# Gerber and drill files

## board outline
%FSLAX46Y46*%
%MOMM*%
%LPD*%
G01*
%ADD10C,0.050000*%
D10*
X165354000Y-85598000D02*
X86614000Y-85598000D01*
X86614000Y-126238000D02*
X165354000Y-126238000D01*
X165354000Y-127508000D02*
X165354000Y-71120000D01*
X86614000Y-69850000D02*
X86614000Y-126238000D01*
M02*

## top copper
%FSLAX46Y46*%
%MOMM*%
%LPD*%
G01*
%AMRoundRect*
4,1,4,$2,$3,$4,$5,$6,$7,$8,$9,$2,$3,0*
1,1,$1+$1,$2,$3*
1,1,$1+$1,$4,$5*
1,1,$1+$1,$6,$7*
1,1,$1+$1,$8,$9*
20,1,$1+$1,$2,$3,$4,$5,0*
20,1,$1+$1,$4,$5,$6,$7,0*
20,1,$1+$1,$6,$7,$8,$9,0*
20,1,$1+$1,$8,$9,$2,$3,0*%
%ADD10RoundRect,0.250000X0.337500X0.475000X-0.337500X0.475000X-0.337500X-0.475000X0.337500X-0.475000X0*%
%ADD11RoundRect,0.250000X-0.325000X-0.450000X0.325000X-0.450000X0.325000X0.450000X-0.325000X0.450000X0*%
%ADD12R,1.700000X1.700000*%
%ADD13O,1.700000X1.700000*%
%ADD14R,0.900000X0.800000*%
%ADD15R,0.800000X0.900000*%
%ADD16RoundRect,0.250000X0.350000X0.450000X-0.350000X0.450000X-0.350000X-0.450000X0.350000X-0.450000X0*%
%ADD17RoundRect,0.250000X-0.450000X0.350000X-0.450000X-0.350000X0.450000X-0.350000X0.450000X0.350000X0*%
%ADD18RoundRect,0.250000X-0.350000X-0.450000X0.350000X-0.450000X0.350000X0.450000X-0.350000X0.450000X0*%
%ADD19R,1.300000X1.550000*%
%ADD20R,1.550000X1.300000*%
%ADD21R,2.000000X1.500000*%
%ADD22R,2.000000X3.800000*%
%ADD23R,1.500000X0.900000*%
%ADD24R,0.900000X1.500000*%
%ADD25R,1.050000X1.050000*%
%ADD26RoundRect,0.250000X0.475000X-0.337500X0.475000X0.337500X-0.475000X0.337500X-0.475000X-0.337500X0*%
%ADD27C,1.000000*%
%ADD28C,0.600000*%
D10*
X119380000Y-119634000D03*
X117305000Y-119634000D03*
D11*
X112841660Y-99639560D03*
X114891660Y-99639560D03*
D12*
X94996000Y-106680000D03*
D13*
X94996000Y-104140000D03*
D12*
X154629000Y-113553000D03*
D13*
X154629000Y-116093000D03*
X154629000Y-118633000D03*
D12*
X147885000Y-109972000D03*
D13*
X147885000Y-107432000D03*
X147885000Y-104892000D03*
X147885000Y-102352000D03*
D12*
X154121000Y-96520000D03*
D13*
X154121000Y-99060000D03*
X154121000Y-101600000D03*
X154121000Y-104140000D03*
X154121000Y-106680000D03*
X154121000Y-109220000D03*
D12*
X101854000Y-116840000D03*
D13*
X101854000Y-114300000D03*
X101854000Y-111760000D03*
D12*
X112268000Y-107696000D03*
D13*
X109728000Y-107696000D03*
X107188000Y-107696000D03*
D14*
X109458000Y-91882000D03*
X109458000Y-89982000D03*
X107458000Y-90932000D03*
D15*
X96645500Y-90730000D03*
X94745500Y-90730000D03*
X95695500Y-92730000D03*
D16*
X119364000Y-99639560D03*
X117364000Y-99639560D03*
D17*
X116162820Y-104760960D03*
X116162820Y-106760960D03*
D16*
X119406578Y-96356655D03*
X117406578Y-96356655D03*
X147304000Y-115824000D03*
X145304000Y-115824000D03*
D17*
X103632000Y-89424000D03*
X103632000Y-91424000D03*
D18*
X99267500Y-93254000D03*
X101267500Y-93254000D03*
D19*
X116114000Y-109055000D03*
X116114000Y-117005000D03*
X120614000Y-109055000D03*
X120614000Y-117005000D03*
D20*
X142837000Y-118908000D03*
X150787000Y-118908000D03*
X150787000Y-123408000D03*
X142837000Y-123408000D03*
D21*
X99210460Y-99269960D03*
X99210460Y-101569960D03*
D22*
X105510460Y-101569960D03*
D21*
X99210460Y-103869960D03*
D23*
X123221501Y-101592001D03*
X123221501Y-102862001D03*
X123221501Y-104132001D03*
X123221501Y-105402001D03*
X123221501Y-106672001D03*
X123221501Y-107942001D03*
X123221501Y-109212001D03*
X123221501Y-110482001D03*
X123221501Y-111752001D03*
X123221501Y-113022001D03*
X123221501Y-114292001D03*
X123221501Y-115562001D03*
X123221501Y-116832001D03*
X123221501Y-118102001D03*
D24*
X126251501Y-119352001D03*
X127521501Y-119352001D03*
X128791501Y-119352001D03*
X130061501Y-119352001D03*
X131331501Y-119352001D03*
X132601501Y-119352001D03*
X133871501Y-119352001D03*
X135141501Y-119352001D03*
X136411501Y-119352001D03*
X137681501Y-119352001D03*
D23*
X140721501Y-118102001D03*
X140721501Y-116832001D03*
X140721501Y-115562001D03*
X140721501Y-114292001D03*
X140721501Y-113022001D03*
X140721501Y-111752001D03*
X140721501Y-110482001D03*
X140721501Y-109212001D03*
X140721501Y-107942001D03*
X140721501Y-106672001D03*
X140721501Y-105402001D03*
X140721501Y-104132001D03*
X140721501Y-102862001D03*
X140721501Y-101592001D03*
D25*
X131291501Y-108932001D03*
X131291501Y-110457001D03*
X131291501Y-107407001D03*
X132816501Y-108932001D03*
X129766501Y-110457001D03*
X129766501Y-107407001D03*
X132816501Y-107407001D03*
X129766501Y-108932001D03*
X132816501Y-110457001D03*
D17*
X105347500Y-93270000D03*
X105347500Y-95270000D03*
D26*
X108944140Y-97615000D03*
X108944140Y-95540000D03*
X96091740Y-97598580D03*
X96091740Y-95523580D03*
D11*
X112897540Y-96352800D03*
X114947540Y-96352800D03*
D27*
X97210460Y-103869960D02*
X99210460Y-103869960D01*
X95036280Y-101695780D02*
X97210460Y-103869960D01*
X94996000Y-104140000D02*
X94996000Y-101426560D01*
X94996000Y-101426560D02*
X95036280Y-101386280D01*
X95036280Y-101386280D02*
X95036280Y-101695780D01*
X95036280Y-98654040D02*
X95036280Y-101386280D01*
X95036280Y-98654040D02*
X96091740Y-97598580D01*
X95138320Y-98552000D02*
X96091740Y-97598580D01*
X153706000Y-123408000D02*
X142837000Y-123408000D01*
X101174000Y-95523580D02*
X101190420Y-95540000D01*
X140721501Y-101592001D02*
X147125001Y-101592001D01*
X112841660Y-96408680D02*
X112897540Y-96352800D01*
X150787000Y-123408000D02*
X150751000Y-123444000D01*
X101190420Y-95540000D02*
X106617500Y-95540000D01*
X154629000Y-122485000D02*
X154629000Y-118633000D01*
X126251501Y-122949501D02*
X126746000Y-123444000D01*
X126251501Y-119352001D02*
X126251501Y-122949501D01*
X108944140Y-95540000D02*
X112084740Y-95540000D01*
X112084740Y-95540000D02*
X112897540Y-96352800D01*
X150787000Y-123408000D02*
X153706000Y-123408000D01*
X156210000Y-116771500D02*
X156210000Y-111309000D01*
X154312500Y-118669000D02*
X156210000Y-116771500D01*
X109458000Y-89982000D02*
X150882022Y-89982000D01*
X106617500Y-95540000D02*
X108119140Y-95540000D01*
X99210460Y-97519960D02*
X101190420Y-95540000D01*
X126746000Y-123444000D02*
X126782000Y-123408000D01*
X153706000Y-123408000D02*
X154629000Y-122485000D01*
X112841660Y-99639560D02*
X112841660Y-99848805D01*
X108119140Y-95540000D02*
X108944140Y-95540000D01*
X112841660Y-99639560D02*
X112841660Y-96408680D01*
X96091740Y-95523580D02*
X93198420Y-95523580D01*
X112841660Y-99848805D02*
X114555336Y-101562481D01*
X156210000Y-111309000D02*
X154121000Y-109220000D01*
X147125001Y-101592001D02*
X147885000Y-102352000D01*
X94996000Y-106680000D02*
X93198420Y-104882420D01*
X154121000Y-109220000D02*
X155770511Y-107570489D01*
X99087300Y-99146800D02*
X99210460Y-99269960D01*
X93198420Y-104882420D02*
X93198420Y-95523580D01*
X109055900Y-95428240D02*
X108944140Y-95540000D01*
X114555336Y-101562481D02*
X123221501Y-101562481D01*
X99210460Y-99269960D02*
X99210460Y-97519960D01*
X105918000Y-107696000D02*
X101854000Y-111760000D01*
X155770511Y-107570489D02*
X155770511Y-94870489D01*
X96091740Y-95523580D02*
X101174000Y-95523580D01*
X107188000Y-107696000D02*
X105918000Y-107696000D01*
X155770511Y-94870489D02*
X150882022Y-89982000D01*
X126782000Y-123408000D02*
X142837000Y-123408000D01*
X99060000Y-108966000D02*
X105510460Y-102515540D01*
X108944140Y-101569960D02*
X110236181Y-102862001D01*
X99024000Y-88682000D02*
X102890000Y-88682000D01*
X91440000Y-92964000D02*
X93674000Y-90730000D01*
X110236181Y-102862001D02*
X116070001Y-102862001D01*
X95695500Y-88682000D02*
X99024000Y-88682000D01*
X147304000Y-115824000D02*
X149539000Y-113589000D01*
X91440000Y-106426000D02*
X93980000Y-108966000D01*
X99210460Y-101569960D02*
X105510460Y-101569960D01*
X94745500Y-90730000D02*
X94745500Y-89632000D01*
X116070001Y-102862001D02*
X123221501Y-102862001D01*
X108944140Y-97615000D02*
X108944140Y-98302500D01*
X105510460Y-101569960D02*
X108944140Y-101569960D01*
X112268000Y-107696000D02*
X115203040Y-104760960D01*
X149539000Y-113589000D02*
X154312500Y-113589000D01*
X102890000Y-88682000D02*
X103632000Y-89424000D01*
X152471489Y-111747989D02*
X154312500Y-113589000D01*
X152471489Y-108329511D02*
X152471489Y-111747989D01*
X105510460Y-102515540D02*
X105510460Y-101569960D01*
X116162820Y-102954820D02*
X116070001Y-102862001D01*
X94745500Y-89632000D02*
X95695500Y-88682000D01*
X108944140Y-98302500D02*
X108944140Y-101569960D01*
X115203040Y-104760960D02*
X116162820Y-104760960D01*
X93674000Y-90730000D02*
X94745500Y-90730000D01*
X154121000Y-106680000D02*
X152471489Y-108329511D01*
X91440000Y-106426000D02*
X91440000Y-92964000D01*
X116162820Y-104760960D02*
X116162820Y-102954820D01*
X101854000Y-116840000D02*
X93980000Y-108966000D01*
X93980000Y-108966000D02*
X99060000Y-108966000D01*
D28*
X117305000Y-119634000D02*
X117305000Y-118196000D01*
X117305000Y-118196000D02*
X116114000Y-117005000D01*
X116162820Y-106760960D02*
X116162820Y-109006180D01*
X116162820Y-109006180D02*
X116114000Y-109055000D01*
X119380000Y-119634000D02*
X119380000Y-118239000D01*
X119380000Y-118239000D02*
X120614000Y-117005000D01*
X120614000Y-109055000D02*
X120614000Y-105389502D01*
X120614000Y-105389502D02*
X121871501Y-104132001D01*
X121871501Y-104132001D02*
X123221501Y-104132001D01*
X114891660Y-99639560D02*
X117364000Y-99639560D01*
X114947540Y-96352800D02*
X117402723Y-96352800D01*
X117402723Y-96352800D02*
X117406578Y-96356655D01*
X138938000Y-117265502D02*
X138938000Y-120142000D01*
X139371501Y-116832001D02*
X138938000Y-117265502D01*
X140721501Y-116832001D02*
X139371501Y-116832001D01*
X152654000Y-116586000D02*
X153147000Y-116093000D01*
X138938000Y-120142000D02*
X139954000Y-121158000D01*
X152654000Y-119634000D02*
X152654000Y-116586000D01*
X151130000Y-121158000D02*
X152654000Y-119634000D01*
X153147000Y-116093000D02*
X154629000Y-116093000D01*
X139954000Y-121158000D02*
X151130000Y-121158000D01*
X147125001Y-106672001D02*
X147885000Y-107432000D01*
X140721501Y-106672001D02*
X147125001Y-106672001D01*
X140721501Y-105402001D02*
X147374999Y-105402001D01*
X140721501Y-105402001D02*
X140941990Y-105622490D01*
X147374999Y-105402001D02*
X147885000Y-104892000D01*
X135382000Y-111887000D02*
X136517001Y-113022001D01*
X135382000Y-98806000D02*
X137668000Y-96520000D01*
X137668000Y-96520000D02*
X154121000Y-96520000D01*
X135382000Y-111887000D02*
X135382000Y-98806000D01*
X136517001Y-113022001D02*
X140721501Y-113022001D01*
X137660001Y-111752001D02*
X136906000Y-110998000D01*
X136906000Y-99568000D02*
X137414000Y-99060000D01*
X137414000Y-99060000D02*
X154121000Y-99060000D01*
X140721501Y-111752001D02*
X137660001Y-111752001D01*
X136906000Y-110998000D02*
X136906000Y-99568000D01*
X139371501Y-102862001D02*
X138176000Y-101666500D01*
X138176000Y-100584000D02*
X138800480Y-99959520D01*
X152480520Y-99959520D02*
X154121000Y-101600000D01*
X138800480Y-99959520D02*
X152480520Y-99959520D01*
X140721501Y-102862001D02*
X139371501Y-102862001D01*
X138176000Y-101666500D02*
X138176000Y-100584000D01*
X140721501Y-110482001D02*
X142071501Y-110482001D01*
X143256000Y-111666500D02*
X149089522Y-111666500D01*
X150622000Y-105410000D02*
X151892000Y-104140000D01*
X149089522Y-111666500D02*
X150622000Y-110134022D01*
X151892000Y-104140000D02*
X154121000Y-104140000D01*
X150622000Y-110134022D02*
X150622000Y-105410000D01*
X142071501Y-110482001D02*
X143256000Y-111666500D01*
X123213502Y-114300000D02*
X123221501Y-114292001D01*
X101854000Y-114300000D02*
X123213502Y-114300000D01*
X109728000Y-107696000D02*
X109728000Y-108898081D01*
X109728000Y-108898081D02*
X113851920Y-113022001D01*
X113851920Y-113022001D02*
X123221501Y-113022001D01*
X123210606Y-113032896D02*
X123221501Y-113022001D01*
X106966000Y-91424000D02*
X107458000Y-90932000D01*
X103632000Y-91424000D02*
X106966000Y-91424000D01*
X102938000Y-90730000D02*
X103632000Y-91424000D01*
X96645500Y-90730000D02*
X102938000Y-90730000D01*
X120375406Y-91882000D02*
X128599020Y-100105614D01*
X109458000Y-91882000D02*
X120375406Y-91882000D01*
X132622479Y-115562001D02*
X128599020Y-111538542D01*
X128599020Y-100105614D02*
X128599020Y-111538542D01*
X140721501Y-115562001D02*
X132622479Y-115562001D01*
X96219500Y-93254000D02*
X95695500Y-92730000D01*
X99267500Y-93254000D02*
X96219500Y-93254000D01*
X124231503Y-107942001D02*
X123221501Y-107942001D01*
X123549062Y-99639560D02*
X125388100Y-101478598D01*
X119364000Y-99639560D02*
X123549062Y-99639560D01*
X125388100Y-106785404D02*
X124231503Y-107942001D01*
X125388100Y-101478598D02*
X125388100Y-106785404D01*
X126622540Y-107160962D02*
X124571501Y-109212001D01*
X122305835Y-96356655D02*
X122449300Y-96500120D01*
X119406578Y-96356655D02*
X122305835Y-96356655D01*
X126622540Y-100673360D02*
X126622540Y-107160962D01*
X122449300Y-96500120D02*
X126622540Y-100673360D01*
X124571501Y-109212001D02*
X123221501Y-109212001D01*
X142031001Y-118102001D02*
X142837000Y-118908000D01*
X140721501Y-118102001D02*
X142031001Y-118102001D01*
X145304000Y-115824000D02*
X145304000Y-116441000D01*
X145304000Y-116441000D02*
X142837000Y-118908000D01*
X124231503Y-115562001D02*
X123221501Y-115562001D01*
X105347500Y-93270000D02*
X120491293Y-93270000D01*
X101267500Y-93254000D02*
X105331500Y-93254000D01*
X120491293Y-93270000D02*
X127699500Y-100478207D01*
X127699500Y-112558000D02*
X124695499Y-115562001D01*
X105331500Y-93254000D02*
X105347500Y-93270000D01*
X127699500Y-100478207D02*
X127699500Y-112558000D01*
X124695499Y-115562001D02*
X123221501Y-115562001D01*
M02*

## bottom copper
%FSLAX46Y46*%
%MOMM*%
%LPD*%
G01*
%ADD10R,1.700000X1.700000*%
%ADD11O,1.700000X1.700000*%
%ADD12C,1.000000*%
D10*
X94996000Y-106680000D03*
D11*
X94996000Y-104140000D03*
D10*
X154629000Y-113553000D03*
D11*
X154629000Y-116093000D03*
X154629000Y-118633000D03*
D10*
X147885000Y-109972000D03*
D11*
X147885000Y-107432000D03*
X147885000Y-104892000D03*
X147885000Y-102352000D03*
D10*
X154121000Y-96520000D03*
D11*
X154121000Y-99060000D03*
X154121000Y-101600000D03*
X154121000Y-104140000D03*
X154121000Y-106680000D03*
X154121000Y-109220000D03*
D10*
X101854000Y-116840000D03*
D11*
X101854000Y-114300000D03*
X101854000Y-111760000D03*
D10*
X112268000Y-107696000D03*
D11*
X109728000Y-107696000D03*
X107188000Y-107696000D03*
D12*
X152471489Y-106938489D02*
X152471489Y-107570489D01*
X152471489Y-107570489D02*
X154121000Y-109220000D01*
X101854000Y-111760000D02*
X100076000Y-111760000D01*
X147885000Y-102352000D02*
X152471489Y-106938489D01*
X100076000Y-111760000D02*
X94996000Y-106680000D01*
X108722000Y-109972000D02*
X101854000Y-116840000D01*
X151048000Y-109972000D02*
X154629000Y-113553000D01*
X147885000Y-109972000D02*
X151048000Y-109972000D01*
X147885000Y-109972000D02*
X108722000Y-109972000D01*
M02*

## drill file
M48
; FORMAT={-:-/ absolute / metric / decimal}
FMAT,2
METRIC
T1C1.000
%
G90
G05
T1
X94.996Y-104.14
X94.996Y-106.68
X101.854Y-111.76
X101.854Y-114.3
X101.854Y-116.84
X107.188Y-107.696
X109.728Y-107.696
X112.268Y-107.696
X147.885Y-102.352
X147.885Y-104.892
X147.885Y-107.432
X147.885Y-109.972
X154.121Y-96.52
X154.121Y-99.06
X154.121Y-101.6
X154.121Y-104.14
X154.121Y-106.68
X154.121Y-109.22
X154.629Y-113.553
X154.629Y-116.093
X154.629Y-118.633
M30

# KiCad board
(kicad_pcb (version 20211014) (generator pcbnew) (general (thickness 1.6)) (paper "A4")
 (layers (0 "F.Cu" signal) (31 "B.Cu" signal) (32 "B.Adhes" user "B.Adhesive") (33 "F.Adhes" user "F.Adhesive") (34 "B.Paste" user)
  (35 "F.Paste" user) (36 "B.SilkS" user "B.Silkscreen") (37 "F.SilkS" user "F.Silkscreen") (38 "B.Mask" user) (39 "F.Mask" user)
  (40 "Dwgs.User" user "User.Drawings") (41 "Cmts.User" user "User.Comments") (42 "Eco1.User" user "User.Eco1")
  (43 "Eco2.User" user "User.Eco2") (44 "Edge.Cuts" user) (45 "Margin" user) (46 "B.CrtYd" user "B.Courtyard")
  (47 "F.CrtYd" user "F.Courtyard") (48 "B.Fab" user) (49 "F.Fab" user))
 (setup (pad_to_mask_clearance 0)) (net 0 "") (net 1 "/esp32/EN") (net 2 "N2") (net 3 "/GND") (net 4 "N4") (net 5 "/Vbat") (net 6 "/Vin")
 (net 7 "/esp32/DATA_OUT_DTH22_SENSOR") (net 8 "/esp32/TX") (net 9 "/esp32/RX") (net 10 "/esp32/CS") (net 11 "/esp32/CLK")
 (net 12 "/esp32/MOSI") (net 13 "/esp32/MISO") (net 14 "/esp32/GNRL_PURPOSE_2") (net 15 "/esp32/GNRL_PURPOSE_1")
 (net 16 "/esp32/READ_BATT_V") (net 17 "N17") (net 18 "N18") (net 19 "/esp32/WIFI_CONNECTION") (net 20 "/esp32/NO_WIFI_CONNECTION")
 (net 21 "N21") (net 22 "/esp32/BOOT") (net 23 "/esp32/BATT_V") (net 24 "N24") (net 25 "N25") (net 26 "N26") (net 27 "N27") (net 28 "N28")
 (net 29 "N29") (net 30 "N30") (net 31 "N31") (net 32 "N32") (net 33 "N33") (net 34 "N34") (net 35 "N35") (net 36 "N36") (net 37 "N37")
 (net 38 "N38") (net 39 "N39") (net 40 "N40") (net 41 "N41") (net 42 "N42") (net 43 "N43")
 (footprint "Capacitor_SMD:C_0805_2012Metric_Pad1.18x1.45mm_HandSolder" (layer "F.Cu") (at 118.3425 119.634 180)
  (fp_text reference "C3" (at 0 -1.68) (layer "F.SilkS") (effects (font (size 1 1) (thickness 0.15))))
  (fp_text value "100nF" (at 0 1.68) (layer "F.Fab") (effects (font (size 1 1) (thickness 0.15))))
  (pad "1" smd roundrect locked (at -1.0375 0 180) (size 1.175 1.45) (layers "F.Cu" "F.Paste" "F.Mask") (roundrect_rratio 0.212766)
   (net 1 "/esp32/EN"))
  (pad "2" smd roundrect locked (at 1.0375 0 180) (size 1.175 1.45) (layers "F.Cu" "F.Paste" "F.Mask") (roundrect_rratio 0.212766)
   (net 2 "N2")))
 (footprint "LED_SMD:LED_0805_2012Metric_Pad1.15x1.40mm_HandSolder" (layer "F.Cu") (at 113.86666 99.63956)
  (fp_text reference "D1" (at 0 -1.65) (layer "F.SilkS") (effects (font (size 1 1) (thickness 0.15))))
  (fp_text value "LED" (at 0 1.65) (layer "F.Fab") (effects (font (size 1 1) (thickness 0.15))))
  (pad "1" smd roundrect locked (at -1.025 0) (size 1.15 1.4) (layers "F.Cu" "F.Paste" "F.Mask") (roundrect_rratio 0.217391) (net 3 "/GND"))
  (pad "2" smd roundrect locked (at 1.025 0) (size 1.15 1.4) (layers "F.Cu" "F.Paste" "F.Mask") (roundrect_rratio 0.217391) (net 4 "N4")))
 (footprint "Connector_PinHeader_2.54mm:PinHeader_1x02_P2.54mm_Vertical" (layer "F.Cu") (at 94.996 106.68 180)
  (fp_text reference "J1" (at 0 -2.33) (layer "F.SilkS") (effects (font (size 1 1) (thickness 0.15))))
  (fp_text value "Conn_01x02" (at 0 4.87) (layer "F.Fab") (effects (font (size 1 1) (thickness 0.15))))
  (pad "1" thru_hole rect locked (at 0 0 180) (size 1.7 1.7) (drill 1) (layers *.Cu *.Mask) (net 3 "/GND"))
  (pad "2" thru_hole oval locked (at 0 2.54 180) (size 1.7 1.7) (drill 1) (layers *.Cu *.Mask) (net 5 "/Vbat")))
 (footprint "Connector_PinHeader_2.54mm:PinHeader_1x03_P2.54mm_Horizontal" (layer "F.Cu") (at 154.629 113.553)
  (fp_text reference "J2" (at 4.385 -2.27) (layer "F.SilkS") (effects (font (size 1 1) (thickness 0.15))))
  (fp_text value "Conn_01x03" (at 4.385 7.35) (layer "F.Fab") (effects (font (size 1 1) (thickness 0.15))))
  (pad "1" thru_hole rect locked (at 0 0) (size 1.7 1.7) (drill 1) (layers *.Cu *.Mask) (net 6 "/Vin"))
  (pad "2" thru_hole oval locked (at 0 2.54) (size 1.7 1.7) (drill 1) (layers *.Cu *.Mask) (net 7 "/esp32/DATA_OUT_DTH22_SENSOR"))
  (pad "3" thru_hole oval locked (at 0 5.08) (size 1.7 1.7) (drill 1) (layers *.Cu *.Mask) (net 3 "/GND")))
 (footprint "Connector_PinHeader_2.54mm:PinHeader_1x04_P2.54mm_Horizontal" (layer "F.Cu") (at 147.885 109.972 180)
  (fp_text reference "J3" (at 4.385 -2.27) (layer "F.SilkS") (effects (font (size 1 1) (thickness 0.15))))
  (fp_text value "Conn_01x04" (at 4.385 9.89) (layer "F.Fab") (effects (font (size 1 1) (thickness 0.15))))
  (pad "1" thru_hole rect locked (at 0 0 180) (size 1.7 1.7) (drill 1) (layers *.Cu *.Mask) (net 6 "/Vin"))
  (pad "2" thru_hole oval locked (at 0 2.54 180) (size 1.7 1.7) (drill 1) (layers *.Cu *.Mask) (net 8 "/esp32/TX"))
  (pad "3" thru_hole oval locked (at 0 5.08 180) (size 1.7 1.7) (drill 1) (layers *.Cu *.Mask) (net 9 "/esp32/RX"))
  (pad "4" thru_hole oval locked (at 0 7.62 180) (size 1.7 1.7) (drill 1) (layers *.Cu *.Mask) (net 3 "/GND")))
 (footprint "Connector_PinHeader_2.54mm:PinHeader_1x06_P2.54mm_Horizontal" (layer "F.Cu") (at 154.121 96.52)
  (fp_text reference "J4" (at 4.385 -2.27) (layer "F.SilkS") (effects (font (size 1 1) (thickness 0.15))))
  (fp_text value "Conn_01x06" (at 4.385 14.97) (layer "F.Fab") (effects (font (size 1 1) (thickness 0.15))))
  (pad "1" thru_hole rect locked (at 0 0) (size 1.7 1.7) (drill 1) (layers *.Cu *.Mask) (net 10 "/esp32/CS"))
  (pad "2" thru_hole oval locked (at 0 2.54) (size 1.7 1.7) (drill 1) (layers *.Cu *.Mask) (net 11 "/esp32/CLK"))
  (pad "3" thru_hole oval locked (at 0 5.08) (size 1.7 1.7) (drill 1) (layers *.Cu *.Mask) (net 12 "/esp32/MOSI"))
  (pad "4" thru_hole oval locked (at 0 7.62) (size 1.7 1.7) (drill 1) (layers *.Cu *.Mask) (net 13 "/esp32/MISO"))
  (pad "5" thru_hole oval locked (at 0 10.16) (size 1.7 1.7) (drill 1) (layers *.Cu *.Mask) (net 6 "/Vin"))
  (pad "6" thru_hole oval locked (at 0 12.7) (size 1.7 1.7) (drill 1) (layers *.Cu *.Mask) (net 3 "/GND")))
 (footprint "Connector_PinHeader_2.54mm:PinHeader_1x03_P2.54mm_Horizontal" (layer "F.Cu") (at 101.854 116.84 180)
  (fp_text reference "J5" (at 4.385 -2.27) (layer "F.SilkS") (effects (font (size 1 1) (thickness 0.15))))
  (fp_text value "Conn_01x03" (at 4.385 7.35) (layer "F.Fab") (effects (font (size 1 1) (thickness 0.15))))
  (pad "1" thru_hole rect locked (at 0 0 180) (size 1.7 1.7) (drill 1) (layers *.Cu *.Mask) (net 6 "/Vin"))
  (pad "2" thru_hole oval locked (at 0 2.54 180) (size 1.7 1.7) (drill 1) (layers *.Cu *.Mask) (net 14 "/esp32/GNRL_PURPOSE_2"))
  (pad "3" thru_hole oval locked (at 0 5.08 180) (size 1.7 1.7) (drill 1) (layers *.Cu *.Mask) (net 3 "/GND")))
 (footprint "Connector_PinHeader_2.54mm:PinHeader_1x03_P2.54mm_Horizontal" (layer "F.Cu") (at 112.268 107.696 -90)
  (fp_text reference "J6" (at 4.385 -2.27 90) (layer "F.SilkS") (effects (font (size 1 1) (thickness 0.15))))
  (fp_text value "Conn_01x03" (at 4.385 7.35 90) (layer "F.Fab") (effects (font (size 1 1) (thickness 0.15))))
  (pad "1" thru_hole rect locked (at 0 0 270) (size 1.7 1.7) (drill 1) (layers *.Cu *.Mask) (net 6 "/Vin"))
  (pad "2" thru_hole oval locked (at 0 2.54 270) (size 1.7 1.7) (drill 1) (layers *.Cu *.Mask) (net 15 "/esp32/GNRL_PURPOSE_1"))
  (pad "3" thru_hole oval locked (at 0 5.08 270) (size 1.7 1.7) (drill 1) (layers *.Cu *.Mask) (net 3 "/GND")))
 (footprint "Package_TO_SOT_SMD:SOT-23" (layer "F.Cu") (at 108.458 90.932 180)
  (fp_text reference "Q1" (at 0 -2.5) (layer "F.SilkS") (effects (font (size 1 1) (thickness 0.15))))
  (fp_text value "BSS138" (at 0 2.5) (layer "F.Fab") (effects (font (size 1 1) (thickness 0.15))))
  (pad "1" smd rect locked (at -1 -0.95 180) (size 0.9 0.8) (layers "F.Cu" "F.Paste" "F.Mask") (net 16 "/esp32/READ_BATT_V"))
  (pad "2" smd rect locked (at -1 0.95 180) (size 0.9 0.8) (layers "F.Cu" "F.Paste" "F.Mask") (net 3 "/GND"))
  (pad "3" smd rect locked (at 1 0 180) (size 0.9 0.8) (layers "F.Cu" "F.Paste" "F.Mask") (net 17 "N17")))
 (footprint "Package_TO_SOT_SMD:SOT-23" (layer "F.Cu") (at 95.6955 91.73 -90)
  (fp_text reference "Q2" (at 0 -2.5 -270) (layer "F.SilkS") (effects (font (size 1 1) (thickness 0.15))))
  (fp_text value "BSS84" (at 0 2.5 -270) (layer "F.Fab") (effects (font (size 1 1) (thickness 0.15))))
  (pad "1" smd rect locked (at -1 -0.95 270) (size 0.9 0.8) (layers "F.Cu" "F.Paste" "F.Mask") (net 17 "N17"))
  (pad "2" smd rect locked (at -1 0.95 270) (size 0.9 0.8) (layers "F.Cu" "F.Paste" "F.Mask") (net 6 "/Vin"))
  (pad "3" smd rect locked (at 1 0 270) (size 0.9 0.8) (layers "F.Cu" "F.Paste" "F.Mask") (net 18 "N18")))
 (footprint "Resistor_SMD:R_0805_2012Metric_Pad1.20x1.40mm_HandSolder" (layer "F.Cu") (at 118.364 99.63956 180)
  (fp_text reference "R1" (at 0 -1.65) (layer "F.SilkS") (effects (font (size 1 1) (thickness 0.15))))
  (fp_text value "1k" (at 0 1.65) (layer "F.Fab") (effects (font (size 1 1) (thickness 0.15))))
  (pad "1" smd roundrect locked (at -1 0 180) (size 1.2 1.4) (layers "F.Cu" "F.Paste" "F.Mask") (roundrect_rratio 0.208333)
   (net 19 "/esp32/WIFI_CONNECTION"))
  (pad "2" smd roundrect locked (at 1 0 180) (size 1.2 1.4) (layers "F.Cu" "F.Paste" "F.Mask") (roundrect_rratio 0.208333) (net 4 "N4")))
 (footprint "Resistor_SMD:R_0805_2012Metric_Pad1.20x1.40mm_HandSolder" (layer "F.Cu") (at 116.16282 105.76096 -90)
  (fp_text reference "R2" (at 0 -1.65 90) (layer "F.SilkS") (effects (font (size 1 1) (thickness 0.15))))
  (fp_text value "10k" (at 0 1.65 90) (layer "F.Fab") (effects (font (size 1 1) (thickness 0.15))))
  (pad "1" smd roundrect locked (at -1 0 270) (size 1.2 1.4) (layers "F.Cu" "F.Paste" "F.Mask") (roundrect_rratio 0.208333) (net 6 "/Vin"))
  (pad "2" smd roundrect locked (at 1 0 270) (size 1.2 1.4) (layers "F.Cu" "F.Paste" "F.Mask") (roundrect_rratio 0.208333) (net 2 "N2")))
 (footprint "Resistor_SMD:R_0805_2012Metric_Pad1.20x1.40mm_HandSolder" (layer "F.Cu") (at 118.406578 96.356655 180)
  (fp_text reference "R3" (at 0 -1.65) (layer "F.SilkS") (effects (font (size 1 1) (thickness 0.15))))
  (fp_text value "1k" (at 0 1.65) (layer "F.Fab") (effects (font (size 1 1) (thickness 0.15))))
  (pad "1" smd roundrect locked (at -1 0 180) (size 1.2 1.4) (layers "F.Cu" "F.Paste" "F.Mask") (roundrect_rratio 0.208333)
   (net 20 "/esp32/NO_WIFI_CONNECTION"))
  (pad "2" smd roundrect locked (at 1 0 180) (size 1.2 1.4) (layers "F.Cu" "F.Paste" "F.Mask") (roundrect_rratio 0.208333) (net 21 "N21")))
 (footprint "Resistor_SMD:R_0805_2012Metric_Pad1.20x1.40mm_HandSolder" (layer "F.Cu") (at 146.304 115.824 180)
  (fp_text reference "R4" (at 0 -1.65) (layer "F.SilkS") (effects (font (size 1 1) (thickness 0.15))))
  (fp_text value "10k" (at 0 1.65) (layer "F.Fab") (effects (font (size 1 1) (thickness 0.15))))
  (pad "1" smd roundrect locked (at -1 0 180) (size 1.2 1.4) (layers "F.Cu" "F.Paste" "F.Mask") (roundrect_rratio 0.208333) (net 6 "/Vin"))
  (pad "2" smd roundrect locked (at 1 0 180) (size 1.2 1.4) (layers "F.Cu" "F.Paste" "F.Mask") (roundrect_rratio 0.208333)
   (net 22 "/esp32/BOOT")))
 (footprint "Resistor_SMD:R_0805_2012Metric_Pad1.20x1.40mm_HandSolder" (layer "F.Cu") (at 103.632 90.424 -90)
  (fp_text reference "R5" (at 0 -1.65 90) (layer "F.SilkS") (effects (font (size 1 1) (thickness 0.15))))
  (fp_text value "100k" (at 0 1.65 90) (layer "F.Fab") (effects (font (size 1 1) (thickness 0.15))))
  (pad "1" smd roundrect locked (at -1 0 270) (size 1.2 1.4) (layers "F.Cu" "F.Paste" "F.Mask") (roundrect_rratio 0.208333) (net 6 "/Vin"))
  (pad "2" smd roundrect locked (at 1 0 270) (size 1.2 1.4) (layers "F.Cu" "F.Paste" "F.Mask") (roundrect_rratio 0.208333) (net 17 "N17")))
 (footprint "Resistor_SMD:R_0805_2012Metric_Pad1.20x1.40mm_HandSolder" (layer "F.Cu") (at 100.2675 93.254)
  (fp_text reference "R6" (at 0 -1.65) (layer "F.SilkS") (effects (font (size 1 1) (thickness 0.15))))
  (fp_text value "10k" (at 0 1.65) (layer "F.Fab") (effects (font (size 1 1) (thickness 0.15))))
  (pad "1" smd roundrect locked (at -1 0) (size 1.2 1.4) (layers "F.Cu" "F.Paste" "F.Mask") (roundrect_rratio 0.208333) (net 18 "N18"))
  (pad "2" smd roundrect locked (at 1 0) (size 1.2 1.4) (layers "F.Cu" "F.Paste" "F.Mask") (roundrect_rratio 0.208333)
   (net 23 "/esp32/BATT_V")))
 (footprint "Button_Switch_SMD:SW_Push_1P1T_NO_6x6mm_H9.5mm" (layer "F.Cu") (at 118.364 113.03 90)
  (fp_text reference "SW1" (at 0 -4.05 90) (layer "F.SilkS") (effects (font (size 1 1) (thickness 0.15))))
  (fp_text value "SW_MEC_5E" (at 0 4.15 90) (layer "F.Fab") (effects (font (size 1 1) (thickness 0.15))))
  (pad "1" smd rect locked (at 3.975 -2.25 90) (size 1.55 1.3) (layers "F.Cu" "F.Paste" "F.Mask") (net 2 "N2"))
  (pad "1" smd rect locked (at -3.975 -2.25 90) (size 1.55 1.3) (layers "F.Cu" "F.Paste" "F.Mask") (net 2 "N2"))
  (pad "2" smd rect locked (at 3.975 2.25 90) (size 1.55 1.3) (layers "F.Cu" "F.Paste" "F.Mask") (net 1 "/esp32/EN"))
  (pad "2" smd rect locked (at -3.975 2.25 90) (size 1.55 1.3) (layers "F.Cu" "F.Paste" "F.Mask") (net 1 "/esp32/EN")))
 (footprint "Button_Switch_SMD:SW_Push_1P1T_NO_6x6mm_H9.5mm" (layer "F.Cu") (at 146.812 121.158)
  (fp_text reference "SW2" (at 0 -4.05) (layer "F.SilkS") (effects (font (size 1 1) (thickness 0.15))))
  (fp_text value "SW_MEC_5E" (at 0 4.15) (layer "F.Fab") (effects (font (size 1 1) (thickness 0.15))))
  (pad "1" smd rect locked (at -3.975 -2.25) (size 1.55 1.3) (layers "F.Cu" "F.Paste" "F.Mask") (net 22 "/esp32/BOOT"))
  (pad "1" smd rect locked (at 3.975 -2.25) (size 1.55 1.3) (layers "F.Cu" "F.Paste" "F.Mask") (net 22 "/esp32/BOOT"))
  (pad "2" smd rect locked (at 3.975 2.25) (size 1.55 1.3) (layers "F.Cu" "F.Paste" "F.Mask") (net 3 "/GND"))
  (pad "2" smd rect locked (at -3.975 2.25) (size 1.55 1.3) (layers "F.Cu" "F.Paste" "F.Mask") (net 3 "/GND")))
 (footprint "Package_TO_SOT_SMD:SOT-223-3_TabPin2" (layer "F.Cu") (at 102.36046 101.56996)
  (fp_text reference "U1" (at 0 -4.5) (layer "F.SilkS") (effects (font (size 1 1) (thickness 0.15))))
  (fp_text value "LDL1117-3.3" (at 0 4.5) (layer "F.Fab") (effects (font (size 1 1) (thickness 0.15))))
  (pad "1" smd rect locked (at -3.15 -2.3) (size 2 1.5) (layers "F.Cu" "F.Paste" "F.Mask") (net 3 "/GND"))
  (pad "2" smd rect locked (at -3.15 0) (size 2 1.5) (layers "F.Cu" "F.Paste" "F.Mask") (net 6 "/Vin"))
  (pad "2" smd rect locked (at 3.15 0) (size 2 3.8) (layers "F.Cu" "F.Paste" "F.Mask") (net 6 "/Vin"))
  (pad "3" smd rect locked (at -3.15 2.3) (size 2 1.5) (layers "F.Cu" "F.Paste" "F.Mask") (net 5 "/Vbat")))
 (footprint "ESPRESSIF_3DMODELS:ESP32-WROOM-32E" (layer "F.Cu") (at 131.971501 108.602001)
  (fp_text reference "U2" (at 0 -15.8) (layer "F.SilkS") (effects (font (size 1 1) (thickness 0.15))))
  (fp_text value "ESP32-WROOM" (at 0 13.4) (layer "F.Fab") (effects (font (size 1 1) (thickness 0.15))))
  (pad "1" smd rect locked (at -8.75 -7.01) (size 1.5 0.9) (layers "F.Cu" "F.Paste" "F.Mask") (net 3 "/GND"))
  (pad "2" smd rect locked (at -8.75 -5.74) (size 1.5 0.9) (layers "F.Cu" "F.Paste" "F.Mask") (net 6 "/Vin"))
  (pad "3" smd rect locked (at -8.75 -4.47) (size 1.5 0.9) (layers "F.Cu" "F.Paste" "F.Mask") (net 1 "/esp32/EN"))
  (pad "4" smd rect locked (at -8.75 -3.2) (size 1.5 0.9) (layers "F.Cu" "F.Paste" "F.Mask") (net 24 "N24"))
  (pad "5" smd rect locked (at -8.75 -1.93) (size 1.5 0.9) (layers "F.Cu" "F.Paste" "F.Mask") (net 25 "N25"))
  (pad "6" smd rect locked (at -8.75 -0.66) (size 1.5 0.9) (layers "F.Cu" "F.Paste" "F.Mask") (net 19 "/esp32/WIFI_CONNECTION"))
  (pad "7" smd rect locked (at -8.75 0.61) (size 1.5 0.9) (layers "F.Cu" "F.Paste" "F.Mask") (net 20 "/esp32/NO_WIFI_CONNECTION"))
  (pad "8" smd rect locked (at -8.75 1.88) (size 1.5 0.9) (layers "F.Cu" "F.Paste" "F.Mask") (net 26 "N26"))
  (pad "9" smd rect locked (at -8.75 3.15) (size 1.5 0.9) (layers "F.Cu" "F.Paste" "F.Mask") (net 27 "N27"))
  (pad "10" smd rect locked (at -8.75 4.42) (size 1.5 0.9) (layers "F.Cu" "F.Paste" "F.Mask") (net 15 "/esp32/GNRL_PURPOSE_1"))
  (pad "11" smd rect locked (at -8.75 5.69) (size 1.5 0.9) (layers "F.Cu" "F.Paste" "F.Mask") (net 14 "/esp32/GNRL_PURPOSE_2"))
  (pad "12" smd rect locked (at -8.75 6.96) (size 1.5 0.9) (layers "F.Cu" "F.Paste" "F.Mask") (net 23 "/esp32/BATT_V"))
  (pad "13" smd rect locked (at -8.75 8.23) (size 1.5 0.9) (layers "F.Cu" "F.Paste" "F.Mask") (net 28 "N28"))
  (pad "14" smd rect locked (at -8.75 9.5) (size 1.5 0.9) (layers "F.Cu" "F.Paste" "F.Mask") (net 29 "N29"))
  (pad "15" smd rect locked (at -5.72 10.75 90) (size 1.5 0.9) (layers "F.Cu" "F.Paste" "F.Mask") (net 3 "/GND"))
  (pad "16" smd rect locked (at -4.45 10.75 90) (size 1.5 0.9) (layers "F.Cu" "F.Paste" "F.Mask") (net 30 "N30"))
  (pad "17" smd rect locked (at -3.18 10.75 90) (size 1.5 0.9) (layers "F.Cu" "F.Paste" "F.Mask") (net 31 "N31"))
  (pad "18" smd rect locked (at -1.91 10.75 90) (size 1.5 0.9) (layers "F.Cu" "F.Paste" "F.Mask") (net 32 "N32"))
  (pad "19" smd rect locked (at -0.64 10.75 90) (size 1.5 0.9) (layers "F.Cu" "F.Paste" "F.Mask") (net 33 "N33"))
  (pad "20" smd rect locked (at 0.63 10.75 90) (size 1.5 0.9) (layers "F.Cu" "F.Paste" "F.Mask") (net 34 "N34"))
  (pad "21" smd rect locked (at 1.9 10.75 90) (size 1.5 0.9) (layers "F.Cu" "F.Paste" "F.Mask") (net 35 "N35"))
  (pad "22" smd rect locked (at 3.17 10.75 90) (size 1.5 0.9) (layers "F.Cu" "F.Paste" "F.Mask") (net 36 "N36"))
  (pad "23" smd rect locked (at 4.44 10.75 90) (size 1.5 0.9) (layers "F.Cu" "F.Paste" "F.Mask") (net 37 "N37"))
  (pad "24" smd rect locked (at 5.71 10.75 90) (size 1.5 0.9) (layers "F.Cu" "F.Paste" "F.Mask") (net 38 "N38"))
  (pad "25" smd rect locked (at 8.75 9.5 180) (size 1.5 0.9) (layers "F.Cu" "F.Paste" "F.Mask") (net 22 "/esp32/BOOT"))
  (pad "26" smd rect locked (at 8.75 8.23 180) (size 1.5 0.9) (layers "F.Cu" "F.Paste" "F.Mask") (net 7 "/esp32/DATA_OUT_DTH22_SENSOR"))
  (pad "27" smd rect locked (at 8.75 6.96 180) (size 1.5 0.9) (layers "F.Cu" "F.Paste" "F.Mask") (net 16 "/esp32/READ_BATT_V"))
  (pad "28" smd rect locked (at 8.75 5.69 180) (size 1.5 0.9) (layers "F.Cu" "F.Paste" "F.Mask") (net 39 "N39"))
  (pad "29" smd rect locked (at 8.75 4.42 180) (size 1.5 0.9) (layers "F.Cu" "F.Paste" "F.Mask") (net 10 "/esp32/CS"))
  (pad "30" smd rect locked (at 8.75 3.15 180) (size 1.5 0.9) (layers "F.Cu" "F.Paste" "F.Mask") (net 11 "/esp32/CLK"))
  (pad "31" smd rect locked (at 8.75 1.88 180) (size 1.5 0.9) (layers "F.Cu" "F.Paste" "F.Mask") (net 13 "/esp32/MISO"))
  (pad "32" smd rect locked (at 8.75 0.61 180) (size 1.5 0.9) (layers "F.Cu" "F.Paste" "F.Mask") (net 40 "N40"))
  (pad "33" smd rect locked (at 8.75 -0.66 180) (size 1.5 0.9) (layers "F.Cu" "F.Paste" "F.Mask") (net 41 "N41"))
  (pad "34" smd rect locked (at 8.75 -1.93 180) (size 1.5 0.9) (layers "F.Cu" "F.Paste" "F.Mask") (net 8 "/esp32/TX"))
  (pad "35" smd rect locked (at 8.75 -3.2 180) (size 1.5 0.9) (layers "F.Cu" "F.Paste" "F.Mask") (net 9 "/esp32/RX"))
  (pad "36" smd rect locked (at 8.75 -4.47 180) (size 1.5 0.9) (layers "F.Cu" "F.Paste" "F.Mask") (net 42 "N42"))
  (pad "37" smd rect locked (at 8.75 -5.74 180) (size 1.5 0.9) (layers "F.Cu" "F.Paste" "F.Mask") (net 12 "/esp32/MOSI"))
  (pad "38" smd rect locked (at 8.75 -7.01 180) (size 1.5 0.9) (layers "F.Cu" "F.Paste" "F.Mask") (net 3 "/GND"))
  (pad "39" smd rect locked (at -0.68 0.33 180) (size 1.05 1.05) (layers "F.Cu" "F.Paste" "F.Mask") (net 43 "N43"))
  (pad "39" smd rect locked (at -0.68 1.855 180) (size 1.05 1.05) (layers "F.Cu" "F.Paste" "F.Mask") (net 43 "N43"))
  (pad "39" smd rect locked (at -0.68 -1.195 180) (size 1.05 1.05) (layers "F.Cu" "F.Paste" "F.Mask") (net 43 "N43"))
  (pad "39" smd rect locked (at 0.845 0.33 180) (size 1.05 1.05) (layers "F.Cu" "F.Paste" "F.Mask") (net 43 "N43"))
  (pad "39" smd rect locked (at -2.205 1.855 180) (size 1.05 1.05) (layers "F.Cu" "F.Paste" "F.Mask") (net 43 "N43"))
  (pad "39" smd rect locked (at -2.205 -1.195 180) (size 1.05 1.05) (layers "F.Cu" "F.Paste" "F.Mask") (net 43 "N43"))
  (pad "39" smd rect locked (at 0.845 -1.195 180) (size 1.05 1.05) (layers "F.Cu" "F.Paste" "F.Mask") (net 43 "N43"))
  (pad "39" smd rect locked (at -2.205 0.33 180) (size 1.05 1.05) (layers "F.Cu" "F.Paste" "F.Mask") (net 43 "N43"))
  (pad "39" smd rect locked (at 0.845 1.855 180) (size 1.05 1.05) (layers "F.Cu" "F.Paste" "F.Mask") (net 43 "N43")))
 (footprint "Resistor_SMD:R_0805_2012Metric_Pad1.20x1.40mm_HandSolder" (layer "F.Cu") (at 105.3475 94.27 -90)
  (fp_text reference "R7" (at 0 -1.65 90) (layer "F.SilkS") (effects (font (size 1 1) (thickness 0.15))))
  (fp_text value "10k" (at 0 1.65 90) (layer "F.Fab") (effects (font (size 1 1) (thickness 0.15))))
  (pad "1" smd roundrect locked (at -1 0 270) (size 1.2 1.4) (layers "F.Cu" "F.Paste" "F.Mask") (roundrect_rratio 0.208333)
   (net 23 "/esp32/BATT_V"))
  (pad "2" smd roundrect locked (at 1 0 270) (size 1.2 1.4) (layers "F.Cu" "F.Paste" "F.Mask") (roundrect_rratio 0.208333) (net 3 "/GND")))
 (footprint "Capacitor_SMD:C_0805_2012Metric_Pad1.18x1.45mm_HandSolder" (layer "F.Cu") (at 108.94414 96.5775 90)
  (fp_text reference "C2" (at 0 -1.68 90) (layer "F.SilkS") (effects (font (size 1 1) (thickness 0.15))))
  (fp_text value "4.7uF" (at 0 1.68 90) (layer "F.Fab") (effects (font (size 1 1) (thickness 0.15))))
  (pad "1" smd roundrect locked (at -1.0375 0 90) (size 1.175 1.45) (layers "F.Cu" "F.Paste" "F.Mask") (roundrect_rratio 0.212766)
   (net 6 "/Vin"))
  (pad "2" smd roundrect locked (at 1.0375 0 90) (size 1.175 1.45) (layers "F.Cu" "F.Paste" "F.Mask") (roundrect_rratio 0.212766)
   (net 3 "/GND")))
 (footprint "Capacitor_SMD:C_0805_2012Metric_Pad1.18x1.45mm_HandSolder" (layer "F.Cu") (at 96.09174 96.56108 90)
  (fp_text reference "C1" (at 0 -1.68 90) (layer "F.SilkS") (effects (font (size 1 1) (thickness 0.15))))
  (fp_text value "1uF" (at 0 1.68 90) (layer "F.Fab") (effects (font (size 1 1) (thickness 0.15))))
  (pad "1" smd roundrect locked (at -1.0375 0 90) (size 1.175 1.45) (layers "F.Cu" "F.Paste" "F.Mask") (roundrect_rratio 0.212766)
   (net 5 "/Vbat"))
  (pad "2" smd roundrect locked (at 1.0375 0 90) (size 1.175 1.45) (layers "F.Cu" "F.Paste" "F.Mask") (roundrect_rratio 0.212766)
   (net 3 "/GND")))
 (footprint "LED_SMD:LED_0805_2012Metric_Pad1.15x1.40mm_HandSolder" (layer "F.Cu") (at 113.92254 96.3528)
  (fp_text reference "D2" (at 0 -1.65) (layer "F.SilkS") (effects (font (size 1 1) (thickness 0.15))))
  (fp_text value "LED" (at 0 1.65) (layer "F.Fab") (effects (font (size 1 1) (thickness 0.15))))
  (pad "1" smd roundrect locked (at -1.025 0) (size 1.15 1.4) (layers "F.Cu" "F.Paste" "F.Mask") (roundrect_rratio 0.217391) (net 3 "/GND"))
  (pad "2" smd roundrect locked (at 1.025 0) (size 1.15 1.4) (layers "F.Cu" "F.Paste" "F.Mask") (roundrect_rratio 0.217391) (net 21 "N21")))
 (gr_line (start 165.354 85.598) (end 86.614 85.598) (layer "Edge.Cuts") (width 0.05))
 (gr_line (start 86.614 126.238) (end 165.354 126.238) (layer "Edge.Cuts") (width 0.05))
 (gr_line (start 165.354 127.508) (end 165.354 71.12) (layer "Edge.Cuts") (width 0.05))
 (gr_line (start 86.614 69.85) (end 86.614 126.238) (layer "Edge.Cuts") (width 0.05))
 (segment (start 97.21046 103.86996) (end 99.21046 103.86996) (width 1) (layer "F.Cu") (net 5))
 (segment (start 95.03628 101.69578) (end 97.21046 103.86996) (width 1) (layer "F.Cu") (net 5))
 (segment (start 94.996 104.14) (end 94.996 101.42656) (width 1) (layer "F.Cu") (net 5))
 (segment (start 94.996 101.42656) (end 95.03628 101.38628) (width 1) (layer "F.Cu") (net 5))
 (segment (start 95.03628 101.38628) (end 95.03628 101.69578) (width 1) (layer "F.Cu") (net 5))
 (segment (start 95.03628 98.65404) (end 95.03628 101.38628) (width 1) (layer "F.Cu") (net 5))
 (segment (start 95.03628 98.65404) (end 96.09174 97.59858) (width 1) (layer "F.Cu") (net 5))
 (segment (start 95.13832 98.552) (end 96.09174 97.59858) (width 1) (layer "F.Cu") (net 5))
 (segment (start 153.706 123.408) (end 142.837 123.408) (width 1) (layer "F.Cu") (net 3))
 (segment (start 101.174 95.52358) (end 101.19042 95.54) (width 1) (layer "F.Cu") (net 3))
 (segment (start 140.721501 101.592001) (end 147.125001 101.592001) (width 1) (layer "F.Cu") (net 3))
 (segment (start 112.84166 96.40868) (end 112.89754 96.3528) (width 1) (layer "F.Cu") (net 3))
 (segment (start 150.787 123.408) (end 150.751 123.444) (width 1) (layer "F.Cu") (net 3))
 (segment (start 101.19042 95.54) (end 106.6175 95.54) (width 1) (layer "F.Cu") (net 3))
 (segment (start 154.629 122.485) (end 154.629 118.633) (width 1) (layer "F.Cu") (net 3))
 (segment (start 126.251501 122.949501) (end 126.746 123.444) (width 1) (layer "F.Cu") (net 3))
 (segment (start 126.251501 119.352001) (end 126.251501 122.949501) (width 1) (layer "F.Cu") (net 3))
 (segment (start 108.94414 95.54) (end 112.08474 95.54) (width 1) (layer "F.Cu") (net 3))
 (segment (start 112.08474 95.54) (end 112.89754 96.3528) (width 1) (layer "F.Cu") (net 3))
 (segment (start 150.787 123.408) (end 153.706 123.408) (width 1) (layer "F.Cu") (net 3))
 (segment (start 156.21 116.7715) (end 156.21 111.309) (width 1) (layer "F.Cu") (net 3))
 (segment (start 154.3125 118.669) (end 156.21 116.7715) (width 1) (layer "F.Cu") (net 3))
 (segment (start 109.458 89.982) (end 150.882022 89.982) (width 1) (layer "F.Cu") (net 3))
 (segment (start 106.6175 95.54) (end 108.11914 95.54) (width 1) (layer "F.Cu") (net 3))
 (segment (start 99.21046 97.51996) (end 101.19042 95.54) (width 1) (layer "F.Cu") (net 3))
 (segment (start 126.746 123.444) (end 126.782 123.408) (width 1) (layer "F.Cu") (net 3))
 (segment (start 153.706 123.408) (end 154.629 122.485) (width 1) (layer "F.Cu") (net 3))
 (segment (start 112.84166 99.63956) (end 112.84166 99.848805) (width 1) (layer "F.Cu") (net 3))
 (segment (start 108.11914 95.54) (end 108.94414 95.54) (width 1) (layer "F.Cu") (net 3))
 (segment (start 112.84166 99.63956) (end 112.84166 96.40868) (width 1) (layer "F.Cu") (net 3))
 (segment (start 96.09174 95.52358) (end 93.19842 95.52358) (width 1) (layer "F.Cu") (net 3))
 (segment (start 112.84166 99.848805) (end 114.555336 101.562481) (width 1) (layer "F.Cu") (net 3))
 (segment (start 156.21 111.309) (end 154.121 109.22) (width 1) (layer "F.Cu") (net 3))
 (segment (start 147.125001 101.592001) (end 147.885 102.352) (width 1) (layer "F.Cu") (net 3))
 (segment (start 94.996 106.68) (end 93.19842 104.88242) (width 1) (layer "F.Cu") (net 3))
 (segment (start 154.121 109.22) (end 155.770511 107.570489) (width 1) (layer "F.Cu") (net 3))
 (segment (start 99.0873 99.1468) (end 99.21046 99.26996) (width 1) (layer "F.Cu") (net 3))
 (segment (start 93.19842 104.88242) (end 93.19842 95.52358) (width 1) (layer "F.Cu") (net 3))
 (segment (start 109.0559 95.42824) (end 108.94414 95.54) (width 1) (layer "F.Cu") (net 3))
 (segment (start 114.555336 101.562481) (end 123.221501 101.562481) (width 1) (layer "F.Cu") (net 3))
 (segment (start 99.21046 99.26996) (end 99.21046 97.51996) (width 1) (layer "F.Cu") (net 3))
 (segment (start 105.918 107.696) (end 101.854 111.76) (width 1) (layer "F.Cu") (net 3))
 (segment (start 155.770511 107.570489) (end 155.770511 94.870489) (width 1) (layer "F.Cu") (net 3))
 (segment (start 96.09174 95.52358) (end 101.174 95.52358) (width 1) (layer "F.Cu") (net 3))
 (segment (start 107.188 107.696) (end 105.918 107.696) (width 1) (layer "F.Cu") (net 3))
 (segment (start 155.770511 94.870489) (end 150.882022 89.982) (width 1) (layer "F.Cu") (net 3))
 (segment (start 126.782 123.408) (end 142.837 123.408) (width 1) (layer "F.Cu") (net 3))
 (segment (start 152.471489 106.938489) (end 152.471489 107.570489) (width 1) (layer "B.Cu") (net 3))
 (segment (start 152.471489 107.570489) (end 154.121 109.22) (width 1) (layer "B.Cu") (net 3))
 (segment (start 101.854 111.76) (end 100.076 111.76) (width 1) (layer "B.Cu") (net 3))
 (segment (start 147.885 102.352) (end 152.471489 106.938489) (width 1) (layer "B.Cu") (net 3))
 (segment (start 100.076 111.76) (end 94.996 106.68) (width 1) (layer "B.Cu") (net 3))
 (segment (start 99.06 108.966) (end 105.51046 102.51554) (width 1) (layer "F.Cu") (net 6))
 (segment (start 108.94414 101.56996) (end 110.236181 102.862001) (width 1) (layer "F.Cu") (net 6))
 (segment (start 99.024 88.682) (end 102.89 88.682) (width 1) (layer "F.Cu") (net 6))
 (segment (start 91.44 92.964) (end 93.674 90.73) (width 1) (layer "F.Cu") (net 6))
 (segment (start 110.236181 102.862001) (end 116.070001 102.862001) (width 1) (layer "F.Cu") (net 6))
 (segment (start 95.6955 88.682) (end 99.024 88.682) (width 1) (layer "F.Cu") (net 6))
 (segment (start 147.304 115.824) (end 149.539 113.589) (width 1) (layer "F.Cu") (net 6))
 (segment (start 91.44 106.426) (end 93.98 108.966) (width 1) (layer "F.Cu") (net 6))
 (segment (start 99.21046 101.56996) (end 105.51046 101.56996) (width 1) (layer "F.Cu") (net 6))
 (segment (start 94.7455 90.73) (end 94.7455 89.632) (width 1) (layer "F.Cu") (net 6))
 (segment (start 116.070001 102.862001) (end 123.221501 102.862001) (width 1) (layer "F.Cu") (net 6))
 (segment (start 108.94414 97.615) (end 108.94414 98.3025) (width 1) (layer "F.Cu") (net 6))
 (segment (start 105.51046 101.56996) (end 108.94414 101.56996) (width 1) (layer "F.Cu") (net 6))
 (segment (start 112.268 107.696) (end 115.20304 104.76096) (width 1) (layer "F.Cu") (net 6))
 (segment (start 149.539 113.589) (end 154.3125 113.589) (width 1) (layer "F.Cu") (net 6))
 (segment (start 102.89 88.682) (end 103.632 89.424) (width 1) (layer "F.Cu") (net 6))
 (segment (start 152.471489 111.747989) (end 154.3125 113.589) (width 1) (layer "F.Cu") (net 6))
 (segment (start 152.471489 108.329511) (end 152.471489 111.747989) (width 1) (layer "F.Cu") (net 6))
 (segment (start 105.51046 102.51554) (end 105.51046 101.56996) (width 1) (layer "F.Cu") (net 6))
 (segment (start 116.16282 102.95482) (end 116.070001 102.862001) (width 1) (layer "F.Cu") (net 6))
 (segment (start 94.7455 89.632) (end 95.6955 88.682) (width 1) (layer "F.Cu") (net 6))
 (segment (start 108.94414 98.3025) (end 108.94414 101.56996) (width 1) (layer "F.Cu") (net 6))
 (segment (start 115.20304 104.76096) (end 116.16282 104.76096) (width 1) (layer "F.Cu") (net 6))
 (segment (start 93.674 90.73) (end 94.7455 90.73) (width 1) (layer "F.Cu") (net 6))
 (segment (start 154.121 106.68) (end 152.471489 108.329511) (width 1) (layer "F.Cu") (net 6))
 (segment (start 91.44 106.426) (end 91.44 92.964) (width 1) (layer "F.Cu") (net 6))
 (segment (start 116.16282 104.76096) (end 116.16282 102.95482) (width 1) (layer "F.Cu") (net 6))
 (segment (start 101.854 116.84) (end 93.98 108.966) (width 1) (layer "F.Cu") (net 6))
 (segment (start 93.98 108.966) (end 99.06 108.966) (width 1) (layer "F.Cu") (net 6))
 (segment (start 108.722 109.972) (end 101.854 116.84) (width 1) (layer "B.Cu") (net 6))
 (segment (start 151.048 109.972) (end 154.629 113.553) (width 1) (layer "B.Cu") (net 6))
 (segment (start 147.885 109.972) (end 151.048 109.972) (width 1) (layer "B.Cu") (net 6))
 (segment (start 147.885 109.972) (end 108.722 109.972) (width 1) (layer "B.Cu") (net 6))
 (segment (start 117.305 119.634) (end 117.305 118.196) (width 0.6) (layer "F.Cu") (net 2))
 (segment (start 117.305 118.196) (end 116.114 117.005) (width 0.6) (layer "F.Cu") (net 2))
 (segment (start 116.16282 106.76096) (end 116.16282 109.00618) (width 0.6) (layer "F.Cu") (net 2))
 (segment (start 116.16282 109.00618) (end 116.114 109.055) (width 0.6) (layer "F.Cu") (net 2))
 (segment (start 119.38 119.634) (end 119.38 118.239) (width 0.6) (layer "F.Cu") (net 1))
 (segment (start 119.38 118.239) (end 120.614 117.005) (width 0.6) (layer "F.Cu") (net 1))
 (segment (start 120.614 109.055) (end 120.614 105.389502) (width 0.6) (layer "F.Cu") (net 1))
 (segment (start 120.614 105.389502) (end 121.871501 104.132001) (width 0.6) (layer "F.Cu") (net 1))
 (segment (start 121.871501 104.132001) (end 123.221501 104.132001) (width 0.6) (layer "F.Cu") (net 1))
 (segment (start 114.89166 99.63956) (end 117.364 99.63956) (width 0.6) (layer "F.Cu") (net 4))
 (segment (start 114.94754 96.3528) (end 117.402723 96.3528) (width 0.6) (layer "F.Cu") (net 21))
 (segment (start 117.402723 96.3528) (end 117.406578 96.356655) (width 0.6) (layer "F.Cu") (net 21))
 (segment (start 138.938 117.265502) (end 138.938 120.142) (width 0.6) (layer "F.Cu") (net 7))
 (segment (start 139.371501 116.832001) (end 138.938 117.265502) (width 0.6) (layer "F.Cu") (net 7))
 (segment (start 140.721501 116.832001) (end 139.371501 116.832001) (width 0.6) (layer "F.Cu") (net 7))
 (segment (start 152.654 116.586) (end 153.147 116.093) (width 0.6) (layer "F.Cu") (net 7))
 (segment (start 138.938 120.142) (end 139.954 121.158) (width 0.6) (layer "F.Cu") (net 7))
 (segment (start 152.654 119.634) (end 152.654 116.586) (width 0.6) (layer "F.Cu") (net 7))
 (segment (start 151.13 121.158) (end 152.654 119.634) (width 0.6) (layer "F.Cu") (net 7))
 (segment (start 153.147 116.093) (end 154.629 116.093) (width 0.6) (layer "F.Cu") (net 7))
 (segment (start 139.954 121.158) (end 151.13 121.158) (width 0.6) (layer "F.Cu") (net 7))
 (segment (start 147.125001 106.672001) (end 147.885 107.432) (width 0.6) (layer "F.Cu") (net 8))
 (segment (start 140.721501 106.672001) (end 147.125001 106.672001) (width 0.6) (layer "F.Cu") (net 8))
 (segment (start 140.721501 105.402001) (end 147.374999 105.402001) (width 0.6) (layer "F.Cu") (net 9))
 (segment (start 140.721501 105.402001) (end 140.94199 105.62249) (width 0.6) (layer "F.Cu") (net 9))
 (segment (start 147.374999 105.402001) (end 147.885 104.892) (width 0.6) (layer "F.Cu") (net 9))
 (segment (start 135.382 111.887) (end 136.517001 113.022001) (width 0.6) (layer "F.Cu") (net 10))
 (segment (start 135.382 98.806) (end 137.668 96.52) (width 0.6) (layer "F.Cu") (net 10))
 (segment (start 137.668 96.52) (end 154.121 96.52) (width 0.6) (layer "F.Cu") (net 10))
 (segment (start 135.382 111.887) (end 135.382 98.806) (width 0.6) (layer "F.Cu") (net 10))
 (segment (start 136.517001 113.022001) (end 140.721501 113.022001) (width 0.6) (layer "F.Cu") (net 10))
 (segment (start 137.660001 111.752001) (end 136.906 110.998) (width 0.6) (layer "F.Cu") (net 11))
 (segment (start 136.906 99.568) (end 137.414 99.06) (width 0.6) (layer "F.Cu") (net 11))
 (segment (start 137.414 99.06) (end 154.121 99.06) (width 0.6) (layer "F.Cu") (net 11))
 (segment (start 140.721501 111.752001) (end 137.660001 111.752001) (width 0.6) (layer "F.Cu") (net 11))
 (segment (start 136.906 110.998) (end 136.906 99.568) (width 0.6) (layer "F.Cu") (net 11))
 (segment (start 139.371501 102.862001) (end 138.176 101.6665) (width 0.6) (layer "F.Cu") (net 12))
 (segment (start 138.176 100.584) (end 138.80048 99.95952) (width 0.6) (layer "F.Cu") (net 12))
 (segment (start 152.48052 99.95952) (end 154.121 101.6) (width 0.6) (layer "F.Cu") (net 12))
 (segment (start 138.80048 99.95952) (end 152.48052 99.95952) (width 0.6) (layer "F.Cu") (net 12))
 (segment (start 140.721501 102.862001) (end 139.371501 102.862001) (width 0.6) (layer "F.Cu") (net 12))
 (segment (start 138.176 101.6665) (end 138.176 100.584) (width 0.6) (layer "F.Cu") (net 12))
 (segment (start 140.721501 110.482001) (end 142.071501 110.482001) (width 0.6) (layer "F.Cu") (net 13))
 (segment (start 143.256 111.6665) (end 149.089522 111.6665) (width 0.6) (layer "F.Cu") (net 13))
 (segment (start 150.622 105.41) (end 151.892 104.14) (width 0.6) (layer "F.Cu") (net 13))
 (segment (start 149.089522 111.6665) (end 150.622 110.134022) (width 0.6) (layer "F.Cu") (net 13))
 (segment (start 151.892 104.14) (end 154.121 104.14) (width 0.6) (layer "F.Cu") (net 13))
 (segment (start 150.622 110.134022) (end 150.622 105.41) (width 0.6) (layer "F.Cu") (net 13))
 (segment (start 142.071501 110.482001) (end 143.256 111.6665) (width 0.6) (layer "F.Cu") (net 13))
 (segment (start 123.213502 114.3) (end 123.221501 114.292001) (width 0.6) (layer "F.Cu") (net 14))
 (segment (start 101.854 114.3) (end 123.213502 114.3) (width 0.6) (layer "F.Cu") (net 14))
 (segment (start 109.728 107.696) (end 109.728 108.898081) (width 0.6) (layer "F.Cu") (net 15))
 (segment (start 109.728 108.898081) (end 113.85192 113.022001) (width 0.6) (layer "F.Cu") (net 15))
 (segment (start 113.85192 113.022001) (end 123.221501 113.022001) (width 0.6) (layer "F.Cu") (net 15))
 (segment (start 123.210606 113.032896) (end 123.221501 113.022001) (width 0.6) (layer "F.Cu") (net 15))
 (segment (start 106.966 91.424) (end 107.458 90.932) (width 0.6) (layer "F.Cu") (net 17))
 (segment (start 103.632 91.424) (end 106.966 91.424) (width 0.6) (layer "F.Cu") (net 17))
 (segment (start 102.938 90.73) (end 103.632 91.424) (width 0.6) (layer "F.Cu") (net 17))
 (segment (start 96.6455 90.73) (end 102.938 90.73) (width 0.6) (layer "F.Cu") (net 17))
 (segment (start 120.375406 91.882) (end 128.59902 100.105614) (width 0.6) (layer "F.Cu") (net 16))
 (segment (start 109.458 91.882) (end 120.375406 91.882) (width 0.6) (layer "F.Cu") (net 16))
 (segment (start 132.622479 115.562001) (end 128.59902 111.538542) (width 0.6) (layer "F.Cu") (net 16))
 (segment (start 128.59902 100.105614) (end 128.59902 111.538542) (width 0.6) (layer "F.Cu") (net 16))
 (segment (start 140.721501 115.562001) (end 132.622479 115.562001) (width 0.6) (layer "F.Cu") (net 16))
 (segment (start 96.2195 93.254) (end 95.6955 92.73) (width 0.6) (layer "F.Cu") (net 18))
 (segment (start 99.2675 93.254) (end 96.2195 93.254) (width 0.6) (layer "F.Cu") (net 18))
 (segment (start 124.231503 107.942001) (end 123.221501 107.942001) (width 0.6) (layer "F.Cu") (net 19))
 (segment (start 123.549062 99.63956) (end 125.3881 101.478598) (width 0.6) (layer "F.Cu") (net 19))
 (segment (start 119.364 99.63956) (end 123.549062 99.63956) (width 0.6) (layer "F.Cu") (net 19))
 (segment (start 125.3881 106.785404) (end 124.231503 107.942001) (width 0.6) (layer "F.Cu") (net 19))
 (segment (start 125.3881 101.478598) (end 125.3881 106.785404) (width 0.6) (layer "F.Cu") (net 19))
 (segment (start 126.62254 107.160962) (end 124.571501 109.212001) (width 0.6) (layer "F.Cu") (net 20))
 (segment (start 122.305835 96.356655) (end 122.4493 96.50012) (width 0.6) (layer "F.Cu") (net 20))
 (segment (start 119.406578 96.356655) (end 122.305835 96.356655) (width 0.6) (layer "F.Cu") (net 20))
 (segment (start 126.62254 100.67336) (end 126.62254 107.160962) (width 0.6) (layer "F.Cu") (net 20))
 (segment (start 122.4493 96.50012) (end 126.62254 100.67336) (width 0.6) (layer "F.Cu") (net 20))
 (segment (start 124.571501 109.212001) (end 123.221501 109.212001) (width 0.6) (layer "F.Cu") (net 20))
 (segment (start 142.031001 118.102001) (end 142.837 118.908) (width 0.6) (layer "F.Cu") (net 22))
 (segment (start 140.721501 118.102001) (end 142.031001 118.102001) (width 0.6) (layer "F.Cu") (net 22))
 (segment (start 145.304 115.824) (end 145.304 116.441) (width 0.6) (layer "F.Cu") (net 22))
 (segment (start 145.304 116.441) (end 142.837 118.908) (width 0.6) (layer "F.Cu") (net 22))
 (segment (start 124.231503 115.562001) (end 123.221501 115.562001) (width 0.6) (layer "F.Cu") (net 23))
 (segment (start 105.3475 93.27) (end 120.491293 93.27) (width 0.6) (layer "F.Cu") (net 23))
 (segment (start 101.2675 93.254) (end 105.3315 93.254) (width 0.6) (layer "F.Cu") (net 23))
 (segment (start 120.491293 93.27) (end 127.6995 100.478207) (width 0.6) (layer "F.Cu") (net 23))
 (segment (start 127.6995 112.558) (end 124.695499 115.562001) (width 0.6) (layer "F.Cu") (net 23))
 (segment (start 105.3315 93.254) (end 105.3475 93.27) (width 0.6) (layer "F.Cu") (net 23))
 (segment (start 127.6995 100.478207) (end 127.6995 112.558) (width 0.6) (layer "F.Cu") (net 23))
 (segment (start 124.695499 115.562001) (end 123.221501 115.562001) (width 0.6) (layer "F.Cu") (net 23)))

